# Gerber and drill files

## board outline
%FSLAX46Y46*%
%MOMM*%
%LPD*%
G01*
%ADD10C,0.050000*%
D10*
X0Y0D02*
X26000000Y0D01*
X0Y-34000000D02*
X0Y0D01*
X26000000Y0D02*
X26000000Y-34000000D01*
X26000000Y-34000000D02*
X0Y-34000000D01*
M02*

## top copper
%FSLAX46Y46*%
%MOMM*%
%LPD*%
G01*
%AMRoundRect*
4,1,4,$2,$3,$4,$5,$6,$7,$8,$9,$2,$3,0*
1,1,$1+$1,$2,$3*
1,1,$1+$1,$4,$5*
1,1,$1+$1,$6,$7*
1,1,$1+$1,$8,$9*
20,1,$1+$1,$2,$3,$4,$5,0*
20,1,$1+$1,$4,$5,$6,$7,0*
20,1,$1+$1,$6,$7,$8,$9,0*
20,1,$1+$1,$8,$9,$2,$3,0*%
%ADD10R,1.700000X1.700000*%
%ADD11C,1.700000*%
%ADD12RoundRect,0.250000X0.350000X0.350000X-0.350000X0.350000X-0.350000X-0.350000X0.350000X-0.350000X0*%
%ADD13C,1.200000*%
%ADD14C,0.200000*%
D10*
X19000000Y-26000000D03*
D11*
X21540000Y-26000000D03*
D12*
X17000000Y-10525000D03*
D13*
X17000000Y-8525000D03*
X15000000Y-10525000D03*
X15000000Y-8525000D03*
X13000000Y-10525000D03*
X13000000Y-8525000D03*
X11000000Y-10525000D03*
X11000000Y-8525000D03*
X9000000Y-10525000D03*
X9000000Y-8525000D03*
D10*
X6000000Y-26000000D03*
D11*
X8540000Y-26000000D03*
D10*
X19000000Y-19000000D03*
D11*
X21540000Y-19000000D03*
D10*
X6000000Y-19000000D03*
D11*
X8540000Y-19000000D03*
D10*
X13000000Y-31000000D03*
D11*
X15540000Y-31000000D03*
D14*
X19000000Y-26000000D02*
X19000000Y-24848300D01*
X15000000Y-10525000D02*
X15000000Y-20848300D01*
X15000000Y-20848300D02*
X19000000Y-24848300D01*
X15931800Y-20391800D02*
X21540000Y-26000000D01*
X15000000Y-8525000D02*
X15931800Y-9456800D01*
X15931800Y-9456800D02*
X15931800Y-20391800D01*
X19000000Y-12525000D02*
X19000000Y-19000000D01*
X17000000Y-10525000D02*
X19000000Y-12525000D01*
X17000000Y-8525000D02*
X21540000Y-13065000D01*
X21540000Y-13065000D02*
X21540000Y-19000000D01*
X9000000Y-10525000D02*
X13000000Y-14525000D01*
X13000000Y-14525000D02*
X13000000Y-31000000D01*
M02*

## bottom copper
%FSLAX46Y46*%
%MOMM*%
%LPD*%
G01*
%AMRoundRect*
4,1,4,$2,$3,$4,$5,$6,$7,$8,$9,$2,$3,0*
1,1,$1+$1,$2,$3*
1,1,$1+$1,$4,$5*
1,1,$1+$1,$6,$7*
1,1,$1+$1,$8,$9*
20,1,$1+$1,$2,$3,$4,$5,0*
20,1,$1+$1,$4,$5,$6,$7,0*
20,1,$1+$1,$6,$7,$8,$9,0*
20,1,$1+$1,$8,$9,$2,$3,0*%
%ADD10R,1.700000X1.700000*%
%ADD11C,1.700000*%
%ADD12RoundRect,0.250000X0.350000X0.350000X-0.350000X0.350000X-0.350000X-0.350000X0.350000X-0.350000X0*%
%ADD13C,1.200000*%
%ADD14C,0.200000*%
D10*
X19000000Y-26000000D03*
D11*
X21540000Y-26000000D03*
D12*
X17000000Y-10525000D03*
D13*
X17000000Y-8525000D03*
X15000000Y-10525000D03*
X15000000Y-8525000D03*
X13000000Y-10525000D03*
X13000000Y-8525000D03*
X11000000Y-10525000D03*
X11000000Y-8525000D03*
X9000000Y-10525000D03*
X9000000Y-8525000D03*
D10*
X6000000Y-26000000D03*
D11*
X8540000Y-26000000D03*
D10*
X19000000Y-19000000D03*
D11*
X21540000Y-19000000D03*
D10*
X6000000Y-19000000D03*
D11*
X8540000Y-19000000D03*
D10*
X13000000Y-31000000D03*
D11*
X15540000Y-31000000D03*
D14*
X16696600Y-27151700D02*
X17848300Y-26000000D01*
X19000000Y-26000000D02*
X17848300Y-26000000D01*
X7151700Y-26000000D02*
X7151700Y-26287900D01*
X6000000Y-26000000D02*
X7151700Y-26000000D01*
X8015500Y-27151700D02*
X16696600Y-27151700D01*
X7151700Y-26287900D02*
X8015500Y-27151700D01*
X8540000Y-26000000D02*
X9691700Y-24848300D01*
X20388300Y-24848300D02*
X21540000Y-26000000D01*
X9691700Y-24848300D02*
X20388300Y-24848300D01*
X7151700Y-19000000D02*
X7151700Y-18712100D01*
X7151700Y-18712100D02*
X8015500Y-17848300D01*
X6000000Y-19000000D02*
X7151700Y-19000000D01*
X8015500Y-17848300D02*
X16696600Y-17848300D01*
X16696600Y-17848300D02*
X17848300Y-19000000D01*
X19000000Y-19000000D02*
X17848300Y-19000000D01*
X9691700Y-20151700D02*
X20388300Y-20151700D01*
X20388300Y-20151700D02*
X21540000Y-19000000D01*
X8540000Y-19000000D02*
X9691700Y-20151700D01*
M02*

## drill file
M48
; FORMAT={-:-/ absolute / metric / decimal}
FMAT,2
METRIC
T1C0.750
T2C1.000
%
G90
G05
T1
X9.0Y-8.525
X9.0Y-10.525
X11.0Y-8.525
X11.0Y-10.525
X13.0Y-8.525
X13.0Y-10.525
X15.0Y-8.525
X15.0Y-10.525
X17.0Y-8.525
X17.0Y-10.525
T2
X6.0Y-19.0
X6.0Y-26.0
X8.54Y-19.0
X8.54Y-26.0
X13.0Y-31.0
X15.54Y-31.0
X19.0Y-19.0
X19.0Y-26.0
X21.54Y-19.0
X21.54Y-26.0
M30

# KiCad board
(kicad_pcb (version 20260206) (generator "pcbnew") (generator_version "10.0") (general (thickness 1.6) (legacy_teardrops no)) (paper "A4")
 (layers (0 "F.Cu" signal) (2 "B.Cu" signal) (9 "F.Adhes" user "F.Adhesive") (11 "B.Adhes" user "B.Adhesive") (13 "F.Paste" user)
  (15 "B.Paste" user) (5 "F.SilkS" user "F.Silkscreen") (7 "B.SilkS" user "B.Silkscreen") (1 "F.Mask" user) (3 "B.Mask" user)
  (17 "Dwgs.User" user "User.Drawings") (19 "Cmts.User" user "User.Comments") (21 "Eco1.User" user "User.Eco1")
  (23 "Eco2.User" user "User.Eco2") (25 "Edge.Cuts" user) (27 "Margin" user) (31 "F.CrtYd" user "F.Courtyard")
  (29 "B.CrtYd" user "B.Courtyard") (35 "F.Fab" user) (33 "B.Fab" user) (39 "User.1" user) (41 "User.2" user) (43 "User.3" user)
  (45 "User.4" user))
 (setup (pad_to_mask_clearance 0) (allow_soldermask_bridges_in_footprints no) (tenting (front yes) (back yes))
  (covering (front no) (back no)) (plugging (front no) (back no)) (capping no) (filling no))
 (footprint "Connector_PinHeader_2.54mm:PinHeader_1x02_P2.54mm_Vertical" (layer "F.Cu") (at 19 26 90)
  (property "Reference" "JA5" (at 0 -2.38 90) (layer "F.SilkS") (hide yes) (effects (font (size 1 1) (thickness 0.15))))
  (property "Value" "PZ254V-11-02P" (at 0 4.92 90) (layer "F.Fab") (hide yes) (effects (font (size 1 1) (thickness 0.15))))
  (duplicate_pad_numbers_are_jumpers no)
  (pad "1" thru_hole rect (at 0 0 90) (size 1.7 1.7) (drill 1) (layers "*.Cu" "*.Mask") (remove_unused_layers no) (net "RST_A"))
  (pad "2" thru_hole circle (at 0 2.54 90) (size 1.7 1.7) (drill 1) (layers "*.Cu" "*.Mask") (remove_unused_layers no) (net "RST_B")))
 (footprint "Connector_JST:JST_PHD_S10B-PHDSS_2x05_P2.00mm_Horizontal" (layer "F.Cu") (at 17 10.525 180)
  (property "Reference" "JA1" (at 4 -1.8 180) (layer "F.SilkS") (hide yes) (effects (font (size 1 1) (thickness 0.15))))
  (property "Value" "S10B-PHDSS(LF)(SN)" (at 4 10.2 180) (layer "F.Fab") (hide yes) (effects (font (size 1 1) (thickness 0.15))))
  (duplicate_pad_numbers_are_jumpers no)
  (pad "1" thru_hole roundrect (at 0 0 180) (size 1.2 1.2) (drill 0.75) (layers "*.Cu" "*.Mask") (remove_unused_layers no)
   (roundrect_rratio 0.208333) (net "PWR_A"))
  (pad "2" thru_hole circle (at 0 2 180) (size 1.2 1.2) (drill 0.75) (layers "*.Cu" "*.Mask") (remove_unused_layers no) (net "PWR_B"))
  (pad "3" thru_hole circle (at 2 0 180) (size 1.2 1.2) (drill 0.75) (layers "*.Cu" "*.Mask") (remove_unused_layers no) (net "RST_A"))
  (pad "4" thru_hole circle (at 2 2 180) (size 1.2 1.2) (drill 0.75) (layers "*.Cu" "*.Mask") (remove_unused_layers no) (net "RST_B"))
  (pad "5" thru_hole circle (at 4 0 180) (size 1.2 1.2) (drill 0.75) (layers "*.Cu" "*.Mask") (remove_unused_layers no))
  (pad "6" thru_hole circle (at 4 2 180) (size 1.2 1.2) (drill 0.75) (layers "*.Cu" "*.Mask") (remove_unused_layers no))
  (pad "7" thru_hole circle (at 6 0 180) (size 1.2 1.2) (drill 0.75) (layers "*.Cu" "*.Mask") (remove_unused_layers no))
  (pad "8" thru_hole circle (at 6 2 180) (size 1.2 1.2) (drill 0.75) (layers "*.Cu" "*.Mask") (remove_unused_layers no))
  (pad "9" thru_hole circle (at 8 0 180) (size 1.2 1.2) (drill 0.75) (layers "*.Cu" "*.Mask") (remove_unused_layers no) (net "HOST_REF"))
  (pad "10" thru_hole circle (at 8 2 180) (size 1.2 1.2) (drill 0.75) (layers "*.Cu" "*.Mask") (remove_unused_layers no)))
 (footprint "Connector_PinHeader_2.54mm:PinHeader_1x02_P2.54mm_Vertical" (layer "F.Cu") (at 6 26 90)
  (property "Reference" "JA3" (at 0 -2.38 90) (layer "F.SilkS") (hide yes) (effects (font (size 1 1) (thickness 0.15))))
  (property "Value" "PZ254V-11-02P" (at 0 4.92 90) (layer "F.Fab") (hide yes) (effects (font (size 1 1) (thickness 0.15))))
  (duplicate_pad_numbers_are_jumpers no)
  (pad "1" thru_hole rect (at 0 0 90) (size 1.7 1.7) (drill 1) (layers "*.Cu" "*.Mask") (remove_unused_layers no) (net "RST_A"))
  (pad "2" thru_hole circle (at 0 2.54 90) (size 1.7 1.7) (drill 1) (layers "*.Cu" "*.Mask") (remove_unused_layers no) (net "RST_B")))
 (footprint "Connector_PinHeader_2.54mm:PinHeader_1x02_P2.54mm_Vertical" (layer "F.Cu") (at 19 19 90)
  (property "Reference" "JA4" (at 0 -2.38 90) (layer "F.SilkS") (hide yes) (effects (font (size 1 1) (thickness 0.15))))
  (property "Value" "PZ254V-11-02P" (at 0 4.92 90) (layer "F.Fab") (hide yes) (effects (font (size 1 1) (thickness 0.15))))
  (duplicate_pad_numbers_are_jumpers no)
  (pad "1" thru_hole rect (at 0 0 90) (size 1.7 1.7) (drill 1) (layers "*.Cu" "*.Mask") (remove_unused_layers no) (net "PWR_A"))
  (pad "2" thru_hole circle (at 0 2.54 90) (size 1.7 1.7) (drill 1) (layers "*.Cu" "*.Mask") (remove_unused_layers no) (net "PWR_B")))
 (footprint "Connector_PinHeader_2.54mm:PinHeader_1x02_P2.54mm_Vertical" (layer "F.Cu") (at 6 19 90)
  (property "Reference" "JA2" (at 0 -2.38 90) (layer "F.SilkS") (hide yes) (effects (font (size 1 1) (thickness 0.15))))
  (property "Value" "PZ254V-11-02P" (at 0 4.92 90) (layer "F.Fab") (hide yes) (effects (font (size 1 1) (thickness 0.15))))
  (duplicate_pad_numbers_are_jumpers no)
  (pad "1" thru_hole rect (at 0 0 90) (size 1.7 1.7) (drill 1) (layers "*.Cu" "*.Mask") (remove_unused_layers no) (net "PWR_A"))
  (pad "2" thru_hole circle (at 0 2.54 90) (size 1.7 1.7) (drill 1) (layers "*.Cu" "*.Mask") (remove_unused_layers no) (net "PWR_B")))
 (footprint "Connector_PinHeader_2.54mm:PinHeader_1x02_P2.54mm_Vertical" (layer "F.Cu") (at 13 31 90)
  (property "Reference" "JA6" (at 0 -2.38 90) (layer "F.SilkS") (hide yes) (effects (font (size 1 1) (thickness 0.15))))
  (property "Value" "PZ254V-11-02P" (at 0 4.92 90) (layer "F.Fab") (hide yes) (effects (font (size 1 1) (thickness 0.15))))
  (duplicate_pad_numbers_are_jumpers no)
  (pad "1" thru_hole rect (at 0 0 90) (size 1.7 1.7) (drill 1) (layers "*.Cu" "*.Mask") (remove_unused_layers no) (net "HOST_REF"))
  (pad "2" thru_hole circle (at 0 2.54 90) (size 1.7 1.7) (drill 1) (layers "*.Cu" "*.Mask") (remove_unused_layers no)))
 (gr_line (start 0 0) (end 26 0) (stroke (width 0.05) (type default)) (layer "Edge.Cuts"))
 (gr_line (start 0 34) (end 0 0) (stroke (width 0.05) (type default)) (layer "Edge.Cuts"))
 (gr_line (start 26 0) (end 26 34) (stroke (width 0.05) (type default)) (layer "Edge.Cuts"))
 (gr_line (start 26 34) (end 0 34) (stroke (width 0.05) (type default)) (layer "Edge.Cuts"))
 (segment (start 19 26) (end 19 24.8483) (width 0.2) (layer "F.Cu") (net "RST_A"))
 (segment (start 15 10.525) (end 15 20.8483) (width 0.2) (layer "F.Cu") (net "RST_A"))
 (segment (start 15 20.8483) (end 19 24.8483) (width 0.2) (layer "F.Cu") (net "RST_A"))
 (segment (start 16.6966 27.1517) (end 17.8483 26) (width 0.2) (layer "B.Cu") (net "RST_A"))
 (segment (start 19 26) (end 17.8483 26) (width 0.2) (layer "B.Cu") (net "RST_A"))
 (segment (start 7.1517 26) (end 7.1517 26.2879) (width 0.2) (layer "B.Cu") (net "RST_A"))
 (segment (start 6 26) (end 7.1517 26) (width 0.2) (layer "B.Cu") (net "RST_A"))
 (segment (start 8.0155 27.1517) (end 16.6966 27.1517) (width 0.2) (layer "B.Cu") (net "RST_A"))
 (segment (start 7.1517 26.2879) (end 8.0155 27.1517) (width 0.2) (layer "B.Cu") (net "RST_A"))
 (segment (start 15.9318 20.3918) (end 21.54 26) (width 0.2) (layer "F.Cu") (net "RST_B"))
 (segment (start 15 8.525) (end 15.9318 9.4568) (width 0.2) (layer "F.Cu") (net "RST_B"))
 (segment (start 15.9318 9.4568) (end 15.9318 20.3918) (width 0.2) (layer "F.Cu") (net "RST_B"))
 (segment (start 8.54 26) (end 9.6917 24.8483) (width 0.2) (layer "B.Cu") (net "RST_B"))
 (segment (start 20.3883 24.8483) (end 21.54 26) (width 0.2) (layer "B.Cu") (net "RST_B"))
 (segment (start 9.6917 24.8483) (end 20.3883 24.8483) (width 0.2) (layer "B.Cu") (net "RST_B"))
 (segment (start 19 12.525) (end 19 19) (width 0.2) (layer "F.Cu") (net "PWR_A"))
 (segment (start 17 10.525) (end 19 12.525) (width 0.2) (layer "F.Cu") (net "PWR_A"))
 (segment (start 7.1517 19) (end 7.1517 18.7121) (width 0.2) (layer "B.Cu") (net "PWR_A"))
 (segment (start 7.1517 18.7121) (end 8.0155 17.8483) (width 0.2) (layer "B.Cu") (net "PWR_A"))
 (segment (start 6 19) (end 7.1517 19) (width 0.2) (layer "B.Cu") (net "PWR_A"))
 (segment (start 8.0155 17.8483) (end 16.6966 17.8483) (width 0.2) (layer "B.Cu") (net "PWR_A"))
 (segment (start 16.6966 17.8483) (end 17.8483 19) (width 0.2) (layer "B.Cu") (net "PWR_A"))
 (segment (start 19 19) (end 17.8483 19) (width 0.2) (layer "B.Cu") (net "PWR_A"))
 (segment (start 17 8.525) (end 21.54 13.065) (width 0.2) (layer "F.Cu") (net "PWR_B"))
 (segment (start 21.54 13.065) (end 21.54 19) (width 0.2) (layer "F.Cu") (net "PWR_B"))
 (segment (start 9.6917 20.1517) (end 20.3883 20.1517) (width 0.2) (layer "B.Cu") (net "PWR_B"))
 (segment (start 20.3883 20.1517) (end 21.54 19) (width 0.2) (layer "B.Cu") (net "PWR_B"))
 (segment (start 8.54 19) (end 9.6917 20.1517) (width 0.2) (layer "B.Cu") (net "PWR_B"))
 (segment (start 9 10.525) (end 13 14.525) (width 0.2) (layer "F.Cu") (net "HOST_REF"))
 (segment (start 13 14.525) (end 13 31) (width 0.2) (layer "F.Cu") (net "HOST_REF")))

